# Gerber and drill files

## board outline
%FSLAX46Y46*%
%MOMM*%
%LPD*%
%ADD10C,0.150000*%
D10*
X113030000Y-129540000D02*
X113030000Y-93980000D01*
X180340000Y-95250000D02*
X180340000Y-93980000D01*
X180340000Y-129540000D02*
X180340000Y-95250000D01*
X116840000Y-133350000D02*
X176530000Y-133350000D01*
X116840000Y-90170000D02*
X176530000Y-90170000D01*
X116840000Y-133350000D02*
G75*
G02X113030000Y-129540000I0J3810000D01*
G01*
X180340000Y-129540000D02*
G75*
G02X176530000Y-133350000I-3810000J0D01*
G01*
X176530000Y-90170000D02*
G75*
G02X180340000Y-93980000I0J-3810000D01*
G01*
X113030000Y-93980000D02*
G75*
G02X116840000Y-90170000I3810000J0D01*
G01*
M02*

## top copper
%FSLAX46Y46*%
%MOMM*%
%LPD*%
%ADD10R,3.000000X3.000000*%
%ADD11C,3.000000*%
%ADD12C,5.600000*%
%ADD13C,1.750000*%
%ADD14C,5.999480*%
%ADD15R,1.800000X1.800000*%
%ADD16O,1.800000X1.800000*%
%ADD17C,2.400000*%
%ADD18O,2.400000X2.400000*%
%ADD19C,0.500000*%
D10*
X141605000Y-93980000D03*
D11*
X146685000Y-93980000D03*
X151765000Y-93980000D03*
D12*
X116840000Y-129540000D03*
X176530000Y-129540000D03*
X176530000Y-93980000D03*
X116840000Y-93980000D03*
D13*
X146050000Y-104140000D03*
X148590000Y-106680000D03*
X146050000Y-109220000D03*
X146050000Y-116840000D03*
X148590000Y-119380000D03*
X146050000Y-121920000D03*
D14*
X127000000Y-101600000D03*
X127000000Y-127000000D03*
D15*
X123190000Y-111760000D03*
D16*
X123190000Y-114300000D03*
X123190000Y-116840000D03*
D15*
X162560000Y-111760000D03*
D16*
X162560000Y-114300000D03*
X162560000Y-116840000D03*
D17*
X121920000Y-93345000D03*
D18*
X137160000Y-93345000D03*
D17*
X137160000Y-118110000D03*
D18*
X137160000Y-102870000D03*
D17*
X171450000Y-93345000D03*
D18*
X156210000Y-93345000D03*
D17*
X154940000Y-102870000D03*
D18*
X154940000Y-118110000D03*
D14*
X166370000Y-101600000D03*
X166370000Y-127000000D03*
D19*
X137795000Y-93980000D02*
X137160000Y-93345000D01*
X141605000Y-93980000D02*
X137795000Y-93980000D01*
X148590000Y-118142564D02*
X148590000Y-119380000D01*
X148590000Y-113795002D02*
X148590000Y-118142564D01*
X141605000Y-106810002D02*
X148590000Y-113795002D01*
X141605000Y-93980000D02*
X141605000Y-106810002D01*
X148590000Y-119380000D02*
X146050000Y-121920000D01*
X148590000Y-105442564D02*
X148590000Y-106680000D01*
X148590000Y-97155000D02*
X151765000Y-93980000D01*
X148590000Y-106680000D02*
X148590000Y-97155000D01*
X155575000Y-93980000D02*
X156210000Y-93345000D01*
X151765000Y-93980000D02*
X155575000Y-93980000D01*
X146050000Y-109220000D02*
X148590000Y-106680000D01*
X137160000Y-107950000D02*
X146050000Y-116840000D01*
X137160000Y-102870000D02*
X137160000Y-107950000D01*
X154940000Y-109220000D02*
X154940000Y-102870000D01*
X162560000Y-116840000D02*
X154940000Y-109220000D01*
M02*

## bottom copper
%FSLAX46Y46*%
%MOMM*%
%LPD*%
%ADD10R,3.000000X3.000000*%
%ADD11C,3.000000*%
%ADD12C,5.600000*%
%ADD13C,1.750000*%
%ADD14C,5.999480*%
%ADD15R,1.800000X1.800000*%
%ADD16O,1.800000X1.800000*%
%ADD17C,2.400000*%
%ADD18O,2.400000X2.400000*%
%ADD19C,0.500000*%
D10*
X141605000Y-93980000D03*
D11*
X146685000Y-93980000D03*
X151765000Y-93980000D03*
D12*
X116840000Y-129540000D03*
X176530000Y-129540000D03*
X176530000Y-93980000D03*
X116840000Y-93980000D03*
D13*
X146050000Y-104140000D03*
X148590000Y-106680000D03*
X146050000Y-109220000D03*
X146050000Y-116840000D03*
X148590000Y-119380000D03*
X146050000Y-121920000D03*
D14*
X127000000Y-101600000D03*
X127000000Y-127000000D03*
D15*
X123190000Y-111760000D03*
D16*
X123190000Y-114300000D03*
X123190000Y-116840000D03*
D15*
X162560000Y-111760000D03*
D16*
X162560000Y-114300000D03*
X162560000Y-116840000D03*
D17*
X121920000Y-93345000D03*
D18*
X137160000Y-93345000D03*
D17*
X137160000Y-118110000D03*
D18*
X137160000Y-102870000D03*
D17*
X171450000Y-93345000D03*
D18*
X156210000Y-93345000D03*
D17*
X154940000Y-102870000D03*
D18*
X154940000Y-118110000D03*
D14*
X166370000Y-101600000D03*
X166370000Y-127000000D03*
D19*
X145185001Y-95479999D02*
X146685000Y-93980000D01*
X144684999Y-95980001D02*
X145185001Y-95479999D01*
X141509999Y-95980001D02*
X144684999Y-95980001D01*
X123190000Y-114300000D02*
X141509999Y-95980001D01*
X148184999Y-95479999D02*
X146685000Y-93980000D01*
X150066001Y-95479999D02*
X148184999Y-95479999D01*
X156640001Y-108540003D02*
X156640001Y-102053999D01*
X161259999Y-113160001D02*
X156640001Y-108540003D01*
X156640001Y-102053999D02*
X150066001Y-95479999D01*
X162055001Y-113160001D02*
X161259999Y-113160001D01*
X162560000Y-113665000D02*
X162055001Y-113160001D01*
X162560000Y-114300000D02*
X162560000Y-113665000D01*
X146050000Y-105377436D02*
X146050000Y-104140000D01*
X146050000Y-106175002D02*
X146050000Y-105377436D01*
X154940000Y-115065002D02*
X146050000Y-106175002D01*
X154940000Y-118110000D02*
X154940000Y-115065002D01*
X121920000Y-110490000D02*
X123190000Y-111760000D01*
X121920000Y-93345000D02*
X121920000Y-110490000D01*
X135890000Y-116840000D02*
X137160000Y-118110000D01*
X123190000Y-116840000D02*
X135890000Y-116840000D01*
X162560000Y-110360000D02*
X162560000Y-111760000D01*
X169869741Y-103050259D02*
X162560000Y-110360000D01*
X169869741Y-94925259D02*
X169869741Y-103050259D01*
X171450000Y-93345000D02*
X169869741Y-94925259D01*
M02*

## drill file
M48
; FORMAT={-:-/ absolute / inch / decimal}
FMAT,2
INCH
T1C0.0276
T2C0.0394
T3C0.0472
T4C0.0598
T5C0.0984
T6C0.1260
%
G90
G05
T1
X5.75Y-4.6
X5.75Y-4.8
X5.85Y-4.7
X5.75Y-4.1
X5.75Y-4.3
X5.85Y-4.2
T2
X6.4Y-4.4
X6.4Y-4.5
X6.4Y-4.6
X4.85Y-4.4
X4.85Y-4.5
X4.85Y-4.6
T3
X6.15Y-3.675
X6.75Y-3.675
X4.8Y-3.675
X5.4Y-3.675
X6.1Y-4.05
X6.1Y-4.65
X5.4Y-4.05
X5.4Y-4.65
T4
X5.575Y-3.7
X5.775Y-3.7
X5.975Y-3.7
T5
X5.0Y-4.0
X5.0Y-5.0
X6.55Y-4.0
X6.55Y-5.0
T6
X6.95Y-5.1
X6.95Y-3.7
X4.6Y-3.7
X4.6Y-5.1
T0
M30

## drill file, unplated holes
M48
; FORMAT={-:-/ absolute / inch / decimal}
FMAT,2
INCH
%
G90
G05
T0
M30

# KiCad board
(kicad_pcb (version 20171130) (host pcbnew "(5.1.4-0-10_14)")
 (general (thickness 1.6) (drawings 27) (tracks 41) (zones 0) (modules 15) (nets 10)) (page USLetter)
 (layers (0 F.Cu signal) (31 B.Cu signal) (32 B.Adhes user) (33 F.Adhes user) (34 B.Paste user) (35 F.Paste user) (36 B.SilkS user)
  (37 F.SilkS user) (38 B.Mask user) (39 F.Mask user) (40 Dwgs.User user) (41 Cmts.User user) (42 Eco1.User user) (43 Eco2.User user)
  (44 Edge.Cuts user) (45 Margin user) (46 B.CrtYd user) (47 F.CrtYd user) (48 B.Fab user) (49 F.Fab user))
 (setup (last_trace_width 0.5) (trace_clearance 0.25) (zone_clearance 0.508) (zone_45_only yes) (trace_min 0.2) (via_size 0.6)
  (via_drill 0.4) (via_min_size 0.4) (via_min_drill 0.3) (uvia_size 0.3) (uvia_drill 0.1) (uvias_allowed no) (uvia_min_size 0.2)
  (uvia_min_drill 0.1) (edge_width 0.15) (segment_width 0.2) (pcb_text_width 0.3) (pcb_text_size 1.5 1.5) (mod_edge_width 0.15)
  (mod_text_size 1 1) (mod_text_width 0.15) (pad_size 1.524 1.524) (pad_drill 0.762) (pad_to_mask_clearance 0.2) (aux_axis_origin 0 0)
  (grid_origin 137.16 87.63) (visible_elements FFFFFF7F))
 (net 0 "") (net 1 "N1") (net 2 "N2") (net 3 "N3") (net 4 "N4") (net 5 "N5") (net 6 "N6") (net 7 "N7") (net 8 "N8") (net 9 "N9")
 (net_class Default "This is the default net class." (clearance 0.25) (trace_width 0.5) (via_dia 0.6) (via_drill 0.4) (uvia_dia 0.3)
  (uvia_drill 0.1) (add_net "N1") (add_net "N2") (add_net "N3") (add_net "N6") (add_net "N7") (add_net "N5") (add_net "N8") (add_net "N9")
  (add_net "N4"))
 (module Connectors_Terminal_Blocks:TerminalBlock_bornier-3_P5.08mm (layer F.Cu) (at 141.605 93.98)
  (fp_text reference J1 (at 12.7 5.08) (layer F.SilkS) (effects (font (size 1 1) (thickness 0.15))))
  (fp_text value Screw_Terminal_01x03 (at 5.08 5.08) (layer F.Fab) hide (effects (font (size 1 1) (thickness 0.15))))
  (pad 1 thru_hole rect (at 0 0) (size 3 3) (drill 1.52) (layers *.Cu *.Mask) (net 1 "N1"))
  (pad 2 thru_hole circle (at 5.08 0) (size 3 3) (drill 1.52) (layers *.Cu *.Mask) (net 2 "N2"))
  (pad 3 thru_hole circle (at 10.16 0) (size 3 3) (drill 1.52) (layers *.Cu *.Mask) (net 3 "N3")))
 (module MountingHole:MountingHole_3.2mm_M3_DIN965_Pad (layer F.Cu) (at 116.84 129.54)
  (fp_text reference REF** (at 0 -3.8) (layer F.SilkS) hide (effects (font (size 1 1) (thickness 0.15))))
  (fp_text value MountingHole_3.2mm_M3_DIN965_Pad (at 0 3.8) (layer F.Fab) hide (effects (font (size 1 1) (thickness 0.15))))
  (pad 1 thru_hole circle (at 0 0) (size 5.6 5.6) (drill 3.2) (layers *.Cu *.Mask)))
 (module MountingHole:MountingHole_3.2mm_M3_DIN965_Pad (layer F.Cu) (at 176.53 129.54)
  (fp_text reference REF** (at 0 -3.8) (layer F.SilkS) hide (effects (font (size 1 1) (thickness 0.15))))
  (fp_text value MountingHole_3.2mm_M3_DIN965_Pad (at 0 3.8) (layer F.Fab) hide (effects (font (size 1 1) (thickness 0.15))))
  (pad 1 thru_hole circle (at 0 0) (size 5.6 5.6) (drill 3.2) (layers *.Cu *.Mask)))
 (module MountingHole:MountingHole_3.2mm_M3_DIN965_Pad (layer F.Cu) (at 176.53 93.98)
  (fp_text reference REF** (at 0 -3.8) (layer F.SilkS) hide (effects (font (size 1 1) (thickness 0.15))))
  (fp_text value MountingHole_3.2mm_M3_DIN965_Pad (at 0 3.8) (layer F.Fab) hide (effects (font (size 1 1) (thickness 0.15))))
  (pad 1 thru_hole circle (at 0 0) (size 5.6 5.6) (drill 3.2) (layers *.Cu *.Mask)))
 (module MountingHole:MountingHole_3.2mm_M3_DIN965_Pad (layer F.Cu) (at 116.84 93.98)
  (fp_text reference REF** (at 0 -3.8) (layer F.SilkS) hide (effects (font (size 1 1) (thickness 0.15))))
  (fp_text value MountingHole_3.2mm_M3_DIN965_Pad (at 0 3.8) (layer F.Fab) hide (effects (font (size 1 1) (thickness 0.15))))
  (pad 1 thru_hole circle (at 0 0) (size 5.6 5.6) (drill 3.2) (layers *.Cu *.Mask)))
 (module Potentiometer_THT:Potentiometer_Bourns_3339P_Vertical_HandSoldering (layer F.Cu) (at 146.05 104.14 180)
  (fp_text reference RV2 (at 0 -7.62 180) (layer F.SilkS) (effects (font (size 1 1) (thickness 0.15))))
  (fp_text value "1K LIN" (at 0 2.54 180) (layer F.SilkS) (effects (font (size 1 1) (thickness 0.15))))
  (pad 1 thru_hole circle (at 0 0 180) (size 1.75 1.75) (drill 0.7) (layers *.Cu *.Mask) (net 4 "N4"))
  (pad 2 thru_hole circle (at -2.54 -2.54 180) (size 1.75 1.75) (drill 0.7) (layers *.Cu *.Mask) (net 3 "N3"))
  (pad 3 thru_hole circle (at 0 -5.08 180) (size 1.75 1.75) (drill 0.7) (layers *.Cu *.Mask) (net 3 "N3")))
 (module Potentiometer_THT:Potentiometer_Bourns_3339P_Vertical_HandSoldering (layer F.Cu) (at 146.05 116.84 180)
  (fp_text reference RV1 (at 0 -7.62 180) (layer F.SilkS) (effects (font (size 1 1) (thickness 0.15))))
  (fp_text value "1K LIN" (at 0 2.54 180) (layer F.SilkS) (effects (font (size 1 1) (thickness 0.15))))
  (pad 1 thru_hole circle (at 0 0 180) (size 1.75 1.75) (drill 0.7) (layers *.Cu *.Mask) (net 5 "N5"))
  (pad 2 thru_hole circle (at -2.54 -2.54 180) (size 1.75 1.75) (drill 0.7) (layers *.Cu *.Mask) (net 1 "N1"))
  (pad 3 thru_hole circle (at 0 -5.08 180) (size 1.75 1.75) (drill 0.7) (layers *.Cu *.Mask) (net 1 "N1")))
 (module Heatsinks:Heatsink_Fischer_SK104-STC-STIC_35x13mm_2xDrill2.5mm (layer F.Cu) (at 127 114.3 90)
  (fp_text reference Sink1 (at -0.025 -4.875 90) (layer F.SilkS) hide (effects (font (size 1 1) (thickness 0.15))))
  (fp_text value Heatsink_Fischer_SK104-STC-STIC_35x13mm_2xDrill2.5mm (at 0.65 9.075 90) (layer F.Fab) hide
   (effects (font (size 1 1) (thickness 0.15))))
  (pad 1 thru_hole circle (at 12.7 0 90) (size 5.99948 5.99948) (drill 2.49936) (layers *.Cu *.Mask))
  (pad 1 thru_hole circle (at -12.7 0 90) (size 5.99948 5.99948) (drill 2.49936) (layers *.Cu *.Mask)))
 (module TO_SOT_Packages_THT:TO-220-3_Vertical (layer F.Cu) (at 123.19 111.76 270)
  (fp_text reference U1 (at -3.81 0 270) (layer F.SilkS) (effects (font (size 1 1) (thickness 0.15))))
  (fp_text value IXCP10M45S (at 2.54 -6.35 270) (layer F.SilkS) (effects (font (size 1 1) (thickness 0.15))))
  (pad 1 thru_hole rect (at 0 0 270) (size 1.8 1.8) (drill 1) (layers *.Cu *.Mask) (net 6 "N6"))
  (pad 2 thru_hole oval (at 2.54 0 270) (size 1.8 1.8) (drill 1) (layers *.Cu *.Mask) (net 2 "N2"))
  (pad 3 thru_hole oval (at 5.08 0 270) (size 1.8 1.8) (drill 1) (layers *.Cu *.Mask) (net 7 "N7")))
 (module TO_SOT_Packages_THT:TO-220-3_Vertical (layer F.Cu) (at 162.56 111.76 270)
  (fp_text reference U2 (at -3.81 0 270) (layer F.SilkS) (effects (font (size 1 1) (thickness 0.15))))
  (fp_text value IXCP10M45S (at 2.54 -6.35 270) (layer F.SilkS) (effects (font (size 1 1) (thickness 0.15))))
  (pad 1 thru_hole rect (at 0 0 270) (size 1.8 1.8) (drill 1) (layers *.Cu *.Mask) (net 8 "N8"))
  (pad 2 thru_hole oval (at 2.54 0 270) (size 1.8 1.8) (drill 1) (layers *.Cu *.Mask) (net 2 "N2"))
  (pad 3 thru_hole oval (at 5.08 0 270) (size 1.8 1.8) (drill 1) (layers *.Cu *.Mask) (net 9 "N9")))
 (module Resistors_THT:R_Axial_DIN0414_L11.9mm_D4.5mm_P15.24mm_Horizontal (layer F.Cu) (at 121.92 93.345)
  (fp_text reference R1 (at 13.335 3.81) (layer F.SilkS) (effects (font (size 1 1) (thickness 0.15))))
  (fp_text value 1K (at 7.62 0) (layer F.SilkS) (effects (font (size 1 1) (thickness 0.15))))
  (pad 1 thru_hole circle (at 0 0) (size 2.4 2.4) (drill 1.2) (layers *.Cu *.Mask) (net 6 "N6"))
  (pad 2 thru_hole oval (at 15.24 0) (size 2.4 2.4) (drill 1.2) (layers *.Cu *.Mask) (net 1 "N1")))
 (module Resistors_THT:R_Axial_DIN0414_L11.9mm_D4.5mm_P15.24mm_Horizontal (layer F.Cu) (at 137.16 118.11 90)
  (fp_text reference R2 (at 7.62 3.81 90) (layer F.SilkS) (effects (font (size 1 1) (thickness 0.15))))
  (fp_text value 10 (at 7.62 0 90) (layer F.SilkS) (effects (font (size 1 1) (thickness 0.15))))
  (pad 1 thru_hole circle (at 0 0 90) (size 2.4 2.4) (drill 1.2) (layers *.Cu *.Mask) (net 7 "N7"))
  (pad 2 thru_hole oval (at 15.24 0 90) (size 2.4 2.4) (drill 1.2) (layers *.Cu *.Mask) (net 5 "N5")))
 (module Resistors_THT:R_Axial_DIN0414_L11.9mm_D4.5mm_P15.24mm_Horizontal (layer F.Cu) (at 171.45 93.345 180)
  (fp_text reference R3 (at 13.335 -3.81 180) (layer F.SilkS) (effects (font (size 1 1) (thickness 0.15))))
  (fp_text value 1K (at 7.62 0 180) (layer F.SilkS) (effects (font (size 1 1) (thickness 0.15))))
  (pad 1 thru_hole circle (at 0 0 180) (size 2.4 2.4) (drill 1.2) (layers *.Cu *.Mask) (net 8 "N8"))
  (pad 2 thru_hole oval (at 15.24 0 180) (size 2.4 2.4) (drill 1.2) (layers *.Cu *.Mask) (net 3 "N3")))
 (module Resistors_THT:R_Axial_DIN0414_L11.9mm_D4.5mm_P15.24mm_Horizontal (layer F.Cu) (at 154.94 102.87 270)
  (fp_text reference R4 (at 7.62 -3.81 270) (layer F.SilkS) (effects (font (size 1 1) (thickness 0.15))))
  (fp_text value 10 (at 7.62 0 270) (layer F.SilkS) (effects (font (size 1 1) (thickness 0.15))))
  (pad 1 thru_hole circle (at 0 0 270) (size 2.4 2.4) (drill 1.2) (layers *.Cu *.Mask) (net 9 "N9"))
  (pad 2 thru_hole oval (at 15.24 0 270) (size 2.4 2.4) (drill 1.2) (layers *.Cu *.Mask) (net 4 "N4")))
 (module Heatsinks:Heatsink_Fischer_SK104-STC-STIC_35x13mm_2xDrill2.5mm (layer F.Cu) (at 166.37 114.3 90)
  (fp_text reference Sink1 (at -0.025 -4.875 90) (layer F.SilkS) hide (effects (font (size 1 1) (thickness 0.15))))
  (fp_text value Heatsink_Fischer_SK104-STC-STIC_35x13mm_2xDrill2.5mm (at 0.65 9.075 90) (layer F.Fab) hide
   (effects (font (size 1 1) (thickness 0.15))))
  (pad 1 thru_hole circle (at 12.7 0 90) (size 5.99948 5.99948) (drill 2.49936) (layers *.Cu *.Mask))
  (pad 1 thru_hole circle (at -12.7 0 90) (size 5.99948 5.99948) (drill 2.49936) (layers *.Cu *.Mask)))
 (gr_line (start 113.03 129.54) (end 113.03 93.98) (layer Edge.Cuts) (width 0.15))
 (gr_line (start 180.34 95.25) (end 180.34 93.98) (layer Edge.Cuts) (width 0.15))
 (gr_line (start 180.34 129.54) (end 180.34 95.25) (layer Edge.Cuts) (width 0.15))
 (gr_line (start 116.84 133.35) (end 176.53 133.35) (layer Edge.Cuts) (width 0.15))
 (gr_line (start 116.84 90.17) (end 176.53 90.17) (layer Edge.Cuts) (width 0.15))
 (gr_arc (start 116.84 129.54) (end 113.03 129.54) (angle -90) (layer Edge.Cuts) (width 0.15))
 (gr_arc (start 176.53 129.54) (end 176.53 133.35) (angle -90) (layer Edge.Cuts) (width 0.15))
 (gr_arc (start 176.53 93.98) (end 180.34 93.98) (angle -90) (layer Edge.Cuts) (width 0.15))
 (gr_arc (start 116.84 93.98) (end 116.84 90.17) (angle -90) (layer Edge.Cuts) (width 0.15))
 (segment (start 137.795 93.98) (end 137.16 93.345) (width 0.5) (layer F.Cu) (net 1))
 (segment (start 141.605 93.98) (end 137.795 93.98) (width 0.5) (layer F.Cu) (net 1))
 (segment (start 148.59 118.142564) (end 148.59 119.38) (width 0.5) (layer F.Cu) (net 1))
 (segment (start 148.59 113.795002) (end 148.59 118.142564) (width 0.5) (layer F.Cu) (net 1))
 (segment (start 141.605 106.810002) (end 148.59 113.795002) (width 0.5) (layer F.Cu) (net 1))
 (segment (start 141.605 93.98) (end 141.605 106.810002) (width 0.5) (layer F.Cu) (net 1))
 (segment (start 148.59 119.38) (end 146.05 121.92) (width 0.5) (layer F.Cu) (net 1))
 (segment (start 145.185001 95.479999) (end 146.685 93.98) (width 0.5) (layer B.Cu) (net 2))
 (segment (start 144.684999 95.980001) (end 145.185001 95.479999) (width 0.5) (layer B.Cu) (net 2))
 (segment (start 141.509999 95.980001) (end 144.684999 95.980001) (width 0.5) (layer B.Cu) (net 2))
 (segment (start 123.19 114.3) (end 141.509999 95.980001) (width 0.5) (layer B.Cu) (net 2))
 (segment (start 148.184999 95.479999) (end 146.685 93.98) (width 0.5) (layer B.Cu) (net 2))
 (segment (start 150.066001 95.479999) (end 148.184999 95.479999) (width 0.5) (layer B.Cu) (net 2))
 (segment (start 156.640001 108.540003) (end 156.640001 102.053999) (width 0.5) (layer B.Cu) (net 2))
 (segment (start 161.259999 113.160001) (end 156.640001 108.540003) (width 0.5) (layer B.Cu) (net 2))
 (segment (start 156.640001 102.053999) (end 150.066001 95.479999) (width 0.5) (layer B.Cu) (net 2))
 (segment (start 162.055001 113.160001) (end 161.259999 113.160001) (width 0.5) (layer B.Cu) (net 2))
 (segment (start 162.56 113.665) (end 162.055001 113.160001) (width 0.5) (layer B.Cu) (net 2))
 (segment (start 162.56 114.3) (end 162.56 113.665) (width 0.5) (layer B.Cu) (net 2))
 (segment (start 148.59 105.442564) (end 148.59 106.68) (width 0.5) (layer F.Cu) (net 3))
 (segment (start 148.59 97.155) (end 151.765 93.98) (width 0.5) (layer F.Cu) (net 3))
 (segment (start 148.59 106.68) (end 148.59 97.155) (width 0.5) (layer F.Cu) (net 3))
 (segment (start 155.575 93.98) (end 156.21 93.345) (width 0.5) (layer F.Cu) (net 3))
 (segment (start 151.765 93.98) (end 155.575 93.98) (width 0.5) (layer F.Cu) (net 3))
 (segment (start 146.05 109.22) (end 148.59 106.68) (width 0.5) (layer F.Cu) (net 3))
 (segment (start 137.16 107.95) (end 146.05 116.84) (width 0.5) (layer F.Cu) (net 5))
 (segment (start 137.16 102.87) (end 137.16 107.95) (width 0.5) (layer F.Cu) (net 5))
 (segment (start 146.05 105.377436) (end 146.05 104.14) (width 0.5) (layer B.Cu) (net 4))
 (segment (start 146.05 106.175002) (end 146.05 105.377436) (width 0.5) (layer B.Cu) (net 4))
 (segment (start 154.94 115.065002) (end 146.05 106.175002) (width 0.5) (layer B.Cu) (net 4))
 (segment (start 154.94 118.11) (end 154.94 115.065002) (width 0.5) (layer B.Cu) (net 4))
 (segment (start 121.92 110.49) (end 123.19 111.76) (width 0.5) (layer B.Cu) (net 6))
 (segment (start 121.92 93.345) (end 121.92 110.49) (width 0.5) (layer B.Cu) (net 6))
 (segment (start 135.89 116.84) (end 137.16 118.11) (width 0.5) (layer B.Cu) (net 7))
 (segment (start 123.19 116.84) (end 135.89 116.84) (width 0.5) (layer B.Cu) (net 7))
 (segment (start 162.56 110.36) (end 162.56 111.76) (width 0.5) (layer B.Cu) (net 8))
 (segment (start 169.869741 103.050259) (end 162.56 110.36) (width 0.5) (layer B.Cu) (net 8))
 (segment (start 169.869741 94.925259) (end 169.869741 103.050259) (width 0.5) (layer B.Cu) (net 8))
 (segment (start 171.45 93.345) (end 169.869741 94.925259) (width 0.5) (layer B.Cu) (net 8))
 (segment (start 154.94 109.22) (end 154.94 102.87) (width 0.5) (layer F.Cu) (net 9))
 (segment (start 162.56 116.84) (end 154.94 109.22) (width 0.5) (layer F.Cu) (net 9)))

